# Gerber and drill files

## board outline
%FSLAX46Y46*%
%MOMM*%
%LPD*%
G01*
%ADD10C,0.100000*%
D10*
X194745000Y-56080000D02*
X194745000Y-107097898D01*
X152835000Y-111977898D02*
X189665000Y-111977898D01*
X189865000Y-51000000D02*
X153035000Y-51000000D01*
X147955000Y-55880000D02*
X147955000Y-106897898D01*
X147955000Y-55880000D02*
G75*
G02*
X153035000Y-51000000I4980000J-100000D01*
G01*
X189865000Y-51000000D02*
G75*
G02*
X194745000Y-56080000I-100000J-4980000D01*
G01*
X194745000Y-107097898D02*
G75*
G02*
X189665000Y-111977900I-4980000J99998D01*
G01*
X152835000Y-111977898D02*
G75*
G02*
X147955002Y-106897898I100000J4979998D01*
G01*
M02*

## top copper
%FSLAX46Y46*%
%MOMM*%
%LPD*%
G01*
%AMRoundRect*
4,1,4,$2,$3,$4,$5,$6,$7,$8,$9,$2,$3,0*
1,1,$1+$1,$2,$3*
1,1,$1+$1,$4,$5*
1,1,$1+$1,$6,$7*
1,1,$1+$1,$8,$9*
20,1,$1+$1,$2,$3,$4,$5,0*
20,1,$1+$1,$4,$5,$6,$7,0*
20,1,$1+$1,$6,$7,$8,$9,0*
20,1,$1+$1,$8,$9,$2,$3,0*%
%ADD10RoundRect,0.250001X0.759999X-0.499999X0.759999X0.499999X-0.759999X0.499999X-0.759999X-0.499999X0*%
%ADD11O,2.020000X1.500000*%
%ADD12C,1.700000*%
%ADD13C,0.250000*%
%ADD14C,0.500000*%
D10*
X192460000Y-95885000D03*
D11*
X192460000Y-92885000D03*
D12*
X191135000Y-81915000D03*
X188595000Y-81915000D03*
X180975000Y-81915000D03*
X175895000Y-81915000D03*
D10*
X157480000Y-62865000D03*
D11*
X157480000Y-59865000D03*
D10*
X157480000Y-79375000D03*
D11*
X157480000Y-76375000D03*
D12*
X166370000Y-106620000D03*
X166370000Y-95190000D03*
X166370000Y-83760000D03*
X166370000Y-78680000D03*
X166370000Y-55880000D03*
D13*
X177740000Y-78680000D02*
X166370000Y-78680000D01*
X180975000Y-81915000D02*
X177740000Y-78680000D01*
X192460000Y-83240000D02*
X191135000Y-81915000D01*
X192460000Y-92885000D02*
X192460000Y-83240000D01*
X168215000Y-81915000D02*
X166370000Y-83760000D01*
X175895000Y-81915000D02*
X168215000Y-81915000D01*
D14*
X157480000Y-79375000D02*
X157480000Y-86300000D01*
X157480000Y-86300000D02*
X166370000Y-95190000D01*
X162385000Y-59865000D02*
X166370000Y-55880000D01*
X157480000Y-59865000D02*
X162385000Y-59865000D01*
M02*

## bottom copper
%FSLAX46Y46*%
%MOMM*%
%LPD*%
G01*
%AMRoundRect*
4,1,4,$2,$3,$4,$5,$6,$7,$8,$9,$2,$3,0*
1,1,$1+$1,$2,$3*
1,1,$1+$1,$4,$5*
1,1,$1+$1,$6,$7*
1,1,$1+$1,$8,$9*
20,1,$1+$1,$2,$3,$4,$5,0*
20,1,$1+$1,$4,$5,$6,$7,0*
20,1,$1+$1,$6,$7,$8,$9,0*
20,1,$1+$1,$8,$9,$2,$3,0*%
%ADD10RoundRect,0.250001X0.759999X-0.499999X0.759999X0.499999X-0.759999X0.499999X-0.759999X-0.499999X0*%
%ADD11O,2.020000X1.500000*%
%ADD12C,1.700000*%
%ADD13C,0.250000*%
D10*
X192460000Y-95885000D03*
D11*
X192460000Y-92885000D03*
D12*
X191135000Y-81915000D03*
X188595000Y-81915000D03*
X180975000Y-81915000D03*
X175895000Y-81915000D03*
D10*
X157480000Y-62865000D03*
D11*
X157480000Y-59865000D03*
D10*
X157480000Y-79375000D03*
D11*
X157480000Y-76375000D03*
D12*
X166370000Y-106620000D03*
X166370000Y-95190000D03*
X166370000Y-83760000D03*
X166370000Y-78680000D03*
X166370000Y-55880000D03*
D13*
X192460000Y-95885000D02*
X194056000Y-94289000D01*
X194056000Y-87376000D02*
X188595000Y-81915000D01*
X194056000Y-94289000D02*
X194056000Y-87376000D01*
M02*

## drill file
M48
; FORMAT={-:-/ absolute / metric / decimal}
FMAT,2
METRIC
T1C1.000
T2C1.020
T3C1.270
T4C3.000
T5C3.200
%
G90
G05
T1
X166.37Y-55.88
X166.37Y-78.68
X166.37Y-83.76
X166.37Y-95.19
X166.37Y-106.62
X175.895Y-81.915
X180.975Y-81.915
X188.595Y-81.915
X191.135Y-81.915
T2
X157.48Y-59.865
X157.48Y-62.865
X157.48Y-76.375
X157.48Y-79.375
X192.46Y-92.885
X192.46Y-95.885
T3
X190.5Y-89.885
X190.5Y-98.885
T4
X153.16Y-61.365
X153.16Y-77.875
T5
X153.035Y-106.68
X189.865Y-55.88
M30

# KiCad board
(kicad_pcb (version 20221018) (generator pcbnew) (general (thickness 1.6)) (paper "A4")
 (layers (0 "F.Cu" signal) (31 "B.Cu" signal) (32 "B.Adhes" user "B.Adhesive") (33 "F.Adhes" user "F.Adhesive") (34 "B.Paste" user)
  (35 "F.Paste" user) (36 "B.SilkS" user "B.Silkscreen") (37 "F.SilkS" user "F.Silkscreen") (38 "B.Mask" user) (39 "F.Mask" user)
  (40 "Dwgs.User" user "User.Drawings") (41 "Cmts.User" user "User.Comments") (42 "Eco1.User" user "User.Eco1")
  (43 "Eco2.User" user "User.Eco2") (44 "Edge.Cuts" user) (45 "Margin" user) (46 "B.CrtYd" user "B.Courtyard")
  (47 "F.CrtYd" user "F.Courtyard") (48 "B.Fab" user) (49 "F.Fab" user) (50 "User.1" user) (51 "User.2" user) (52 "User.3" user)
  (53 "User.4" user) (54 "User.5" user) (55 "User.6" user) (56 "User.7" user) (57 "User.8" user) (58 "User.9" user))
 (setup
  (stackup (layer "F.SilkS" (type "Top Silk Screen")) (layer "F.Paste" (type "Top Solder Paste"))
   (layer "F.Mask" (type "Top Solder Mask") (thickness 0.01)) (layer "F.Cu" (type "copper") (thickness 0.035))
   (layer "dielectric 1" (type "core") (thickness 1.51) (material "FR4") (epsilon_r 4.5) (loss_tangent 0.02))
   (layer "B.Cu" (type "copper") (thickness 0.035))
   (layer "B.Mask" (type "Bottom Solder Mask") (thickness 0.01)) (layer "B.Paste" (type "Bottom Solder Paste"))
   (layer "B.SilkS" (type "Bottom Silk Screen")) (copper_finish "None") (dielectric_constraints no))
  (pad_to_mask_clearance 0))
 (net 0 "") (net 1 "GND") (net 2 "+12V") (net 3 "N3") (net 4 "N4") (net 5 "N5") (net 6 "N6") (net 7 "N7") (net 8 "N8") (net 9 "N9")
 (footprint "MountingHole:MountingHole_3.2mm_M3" (layer "F.Cu") (at 153.035 106.68)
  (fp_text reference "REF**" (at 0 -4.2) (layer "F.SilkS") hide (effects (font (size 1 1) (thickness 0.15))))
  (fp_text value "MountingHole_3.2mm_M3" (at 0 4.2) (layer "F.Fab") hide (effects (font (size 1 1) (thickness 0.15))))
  (pad "" np_thru_hole circle (at 0 0) (size 3.2 3.2) (drill 3.2) (layers "*.Cu" "*.Mask")))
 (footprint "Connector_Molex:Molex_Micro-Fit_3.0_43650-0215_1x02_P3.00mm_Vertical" (layer "F.Cu") (at 192.46 95.885 90)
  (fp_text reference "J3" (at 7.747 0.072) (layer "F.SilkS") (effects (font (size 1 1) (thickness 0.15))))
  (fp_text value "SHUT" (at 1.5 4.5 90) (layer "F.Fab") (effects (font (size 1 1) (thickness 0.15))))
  (pad "" np_thru_hole circle (at -3 -1.96 90) (size 1.27 1.27) (drill 1.27) (layers "*.Cu" "*.Mask"))
  (pad "" np_thru_hole circle (at 6 -1.96 90) (size 1.27 1.27) (drill 1.27) (layers "*.Cu" "*.Mask"))
  (pad "1" thru_hole roundrect (at 0 0 90) (size 1.5 2.02) (drill 1.02) (layers "*.Cu" "*.Mask") (roundrect_rratio 0.166667) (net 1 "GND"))
  (pad "2" thru_hole oval (at 3 0 90) (size 1.5 2.02) (drill 1.02) (layers "*.Cu" "*.Mask") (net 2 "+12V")))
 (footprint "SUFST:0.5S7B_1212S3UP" (layer "F.Cu") (at 183.265 81.915 180)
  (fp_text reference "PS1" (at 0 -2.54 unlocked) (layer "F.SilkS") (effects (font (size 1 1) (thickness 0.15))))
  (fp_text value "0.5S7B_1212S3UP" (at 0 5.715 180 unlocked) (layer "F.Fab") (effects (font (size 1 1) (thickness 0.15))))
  (pad "1" thru_hole circle (at -7.87 0 180) (size 1.7 1.7) (drill 1) (layers "*.Cu" "*.Mask") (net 2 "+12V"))
  (pad "2" thru_hole circle (at -5.33 0 180) (size 1.7 1.7) (drill 1) (layers "*.Cu" "*.Mask") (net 1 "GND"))
  (pad "5" thru_hole circle (at 2.29 0 180) (size 1.7 1.7) (drill 1) (layers "*.Cu" "*.Mask") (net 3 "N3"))
  (pad "7" thru_hole circle (at 7.37 0 180) (size 1.7 1.7) (drill 1) (layers "*.Cu" "*.Mask") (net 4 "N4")))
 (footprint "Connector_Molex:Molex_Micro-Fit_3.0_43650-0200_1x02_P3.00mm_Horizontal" (layer "F.Cu") (at 157.48 62.865 90)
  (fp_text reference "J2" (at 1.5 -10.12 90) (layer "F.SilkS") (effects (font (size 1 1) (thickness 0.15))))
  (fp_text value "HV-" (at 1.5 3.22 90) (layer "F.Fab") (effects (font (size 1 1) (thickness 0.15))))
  (pad "" np_thru_hole circle (at 1.5 -4.32 90) (size 3 3) (drill 3) (layers "*.Cu" "*.Mask"))
  (pad "1" thru_hole roundrect (at 0 0 90) (size 1.5 2.02) (drill 1.02) (layers "*.Cu" "*.Mask") (roundrect_rratio 0.166667) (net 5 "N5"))
  (pad "2" thru_hole oval (at 3 0 90) (size 1.5 2.02) (drill 1.02) (layers "*.Cu" "*.Mask") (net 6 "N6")))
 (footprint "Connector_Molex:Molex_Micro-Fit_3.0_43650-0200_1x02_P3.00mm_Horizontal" (layer "F.Cu") (at 157.48 79.375 90)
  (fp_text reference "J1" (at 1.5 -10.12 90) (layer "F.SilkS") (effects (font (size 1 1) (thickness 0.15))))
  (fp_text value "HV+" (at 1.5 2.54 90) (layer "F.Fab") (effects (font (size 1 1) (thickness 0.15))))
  (pad "" np_thru_hole circle (at 1.5 -4.32 90) (size 3 3) (drill 3) (layers "*.Cu" "*.Mask"))
  (pad "1" thru_hole roundrect (at 0 0 90) (size 1.5 2.02) (drill 1.02) (layers "*.Cu" "*.Mask") (roundrect_rratio 0.166667) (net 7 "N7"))
  (pad "2" thru_hole oval (at 3 0 90) (size 1.5 2.02) (drill 1.02) (layers "*.Cu" "*.Mask") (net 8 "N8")))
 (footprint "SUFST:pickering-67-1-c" (layer "F.Cu") (at 166.37 81.22 90)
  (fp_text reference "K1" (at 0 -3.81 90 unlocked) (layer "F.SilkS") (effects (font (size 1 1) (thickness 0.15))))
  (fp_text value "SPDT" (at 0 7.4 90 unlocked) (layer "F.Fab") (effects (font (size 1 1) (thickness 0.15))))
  (pad "1" thru_hole circle (at -25.4 0 90) (size 1.7 1.7) (drill 1) (layers "*.Cu" "*.Mask") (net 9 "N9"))
  (pad "2" thru_hole circle (at -13.97 0 90) (size 1.7 1.7) (drill 1) (layers "*.Cu" "*.Mask") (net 7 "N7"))
  (pad "3" thru_hole circle (at -2.54 0 90) (size 1.7 1.7) (drill 1) (layers "*.Cu" "*.Mask") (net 4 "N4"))
  (pad "5" thru_hole circle (at 2.54 0 90) (size 1.7 1.7) (drill 1) (layers "*.Cu" "*.Mask") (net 3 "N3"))
  (pad "7" thru_hole circle (at 25.34 0 90) (size 1.7 1.7) (drill 1) (layers "*.Cu" "*.Mask") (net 6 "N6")))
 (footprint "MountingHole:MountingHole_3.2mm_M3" (layer "F.Cu") (at 189.865 55.88)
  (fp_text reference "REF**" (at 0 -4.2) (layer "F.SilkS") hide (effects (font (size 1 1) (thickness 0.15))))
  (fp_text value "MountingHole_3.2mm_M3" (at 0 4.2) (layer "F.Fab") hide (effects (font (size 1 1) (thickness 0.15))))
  (pad "" np_thru_hole circle (at 0 0) (size 3.2 3.2) (drill 3.2) (layers "*.Cu" "*.Mask")))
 (gr_line (start 194.745 56.08) (end 194.745 107.097898) (stroke (width 0.1) (type default)) (layer "Edge.Cuts"))
 (gr_line (start 152.835 111.977898) (end 189.665 111.977898) (stroke (width 0.1) (type default)) (layer "Edge.Cuts"))
 (gr_line (start 189.865 51) (end 153.035 51) (stroke (width 0.1) (type default)) (layer "Edge.Cuts"))
 (gr_line (start 147.955 55.88) (end 147.955 106.897898) (stroke (width 0.1) (type default)) (layer "Edge.Cuts"))
 (gr_arc (start 147.955 55.88) (mid 149.484319 52.387898) (end 153.035 51) (stroke (width 0.1) (type default)) (layer "Edge.Cuts"))
 (gr_arc (start 189.865 51) (mid 193.357102 52.529319) (end 194.745 56.08) (stroke (width 0.1) (type default)) (layer "Edge.Cuts"))
 (gr_arc (start 194.745 107.097898) (mid 193.215681 110.59) (end 189.665 111.977898) (stroke (width 0.1) (type default)) (layer "Edge.Cuts"))
 (gr_arc (start 152.835 111.977898) (mid 149.342898 110.448579) (end 147.955 106.897898) (stroke (width 0.1) (type default))
  (layer "Edge.Cuts"))
 (segment (start 177.74 78.68) (end 166.37 78.68) (width 0.25) (layer "F.Cu") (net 3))
 (segment (start 180.975 81.915) (end 177.74 78.68) (width 0.25) (layer "F.Cu") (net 3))
 (segment (start 192.46 95.885) (end 194.056 94.289) (width 0.25) (layer "B.Cu") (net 1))
 (segment (start 194.056 87.376) (end 188.595 81.915) (width 0.25) (layer "B.Cu") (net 1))
 (segment (start 194.056 94.289) (end 194.056 87.376) (width 0.25) (layer "B.Cu") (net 1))
 (segment (start 192.46 83.24) (end 191.135 81.915) (width 0.25) (layer "F.Cu") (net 2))
 (segment (start 192.46 92.885) (end 192.46 83.24) (width 0.25) (layer "F.Cu") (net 2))
 (segment (start 168.215 81.915) (end 166.37 83.76) (width 0.25) (layer "F.Cu") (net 4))
 (segment (start 175.895 81.915) (end 168.215 81.915) (width 0.25) (layer "F.Cu") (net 4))
 (segment (start 157.48 79.375) (end 157.48 86.3) (width 0.5) (layer "F.Cu") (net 7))
 (segment (start 157.48 86.3) (end 166.37 95.19) (width 0.5) (layer "F.Cu") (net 7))
 (segment (start 162.385 59.865) (end 166.37 55.88) (width 0.5) (layer "F.Cu") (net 6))
 (segment (start 157.48 59.865) (end 162.385 59.865) (width 0.5) (layer "F.Cu") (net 6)))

